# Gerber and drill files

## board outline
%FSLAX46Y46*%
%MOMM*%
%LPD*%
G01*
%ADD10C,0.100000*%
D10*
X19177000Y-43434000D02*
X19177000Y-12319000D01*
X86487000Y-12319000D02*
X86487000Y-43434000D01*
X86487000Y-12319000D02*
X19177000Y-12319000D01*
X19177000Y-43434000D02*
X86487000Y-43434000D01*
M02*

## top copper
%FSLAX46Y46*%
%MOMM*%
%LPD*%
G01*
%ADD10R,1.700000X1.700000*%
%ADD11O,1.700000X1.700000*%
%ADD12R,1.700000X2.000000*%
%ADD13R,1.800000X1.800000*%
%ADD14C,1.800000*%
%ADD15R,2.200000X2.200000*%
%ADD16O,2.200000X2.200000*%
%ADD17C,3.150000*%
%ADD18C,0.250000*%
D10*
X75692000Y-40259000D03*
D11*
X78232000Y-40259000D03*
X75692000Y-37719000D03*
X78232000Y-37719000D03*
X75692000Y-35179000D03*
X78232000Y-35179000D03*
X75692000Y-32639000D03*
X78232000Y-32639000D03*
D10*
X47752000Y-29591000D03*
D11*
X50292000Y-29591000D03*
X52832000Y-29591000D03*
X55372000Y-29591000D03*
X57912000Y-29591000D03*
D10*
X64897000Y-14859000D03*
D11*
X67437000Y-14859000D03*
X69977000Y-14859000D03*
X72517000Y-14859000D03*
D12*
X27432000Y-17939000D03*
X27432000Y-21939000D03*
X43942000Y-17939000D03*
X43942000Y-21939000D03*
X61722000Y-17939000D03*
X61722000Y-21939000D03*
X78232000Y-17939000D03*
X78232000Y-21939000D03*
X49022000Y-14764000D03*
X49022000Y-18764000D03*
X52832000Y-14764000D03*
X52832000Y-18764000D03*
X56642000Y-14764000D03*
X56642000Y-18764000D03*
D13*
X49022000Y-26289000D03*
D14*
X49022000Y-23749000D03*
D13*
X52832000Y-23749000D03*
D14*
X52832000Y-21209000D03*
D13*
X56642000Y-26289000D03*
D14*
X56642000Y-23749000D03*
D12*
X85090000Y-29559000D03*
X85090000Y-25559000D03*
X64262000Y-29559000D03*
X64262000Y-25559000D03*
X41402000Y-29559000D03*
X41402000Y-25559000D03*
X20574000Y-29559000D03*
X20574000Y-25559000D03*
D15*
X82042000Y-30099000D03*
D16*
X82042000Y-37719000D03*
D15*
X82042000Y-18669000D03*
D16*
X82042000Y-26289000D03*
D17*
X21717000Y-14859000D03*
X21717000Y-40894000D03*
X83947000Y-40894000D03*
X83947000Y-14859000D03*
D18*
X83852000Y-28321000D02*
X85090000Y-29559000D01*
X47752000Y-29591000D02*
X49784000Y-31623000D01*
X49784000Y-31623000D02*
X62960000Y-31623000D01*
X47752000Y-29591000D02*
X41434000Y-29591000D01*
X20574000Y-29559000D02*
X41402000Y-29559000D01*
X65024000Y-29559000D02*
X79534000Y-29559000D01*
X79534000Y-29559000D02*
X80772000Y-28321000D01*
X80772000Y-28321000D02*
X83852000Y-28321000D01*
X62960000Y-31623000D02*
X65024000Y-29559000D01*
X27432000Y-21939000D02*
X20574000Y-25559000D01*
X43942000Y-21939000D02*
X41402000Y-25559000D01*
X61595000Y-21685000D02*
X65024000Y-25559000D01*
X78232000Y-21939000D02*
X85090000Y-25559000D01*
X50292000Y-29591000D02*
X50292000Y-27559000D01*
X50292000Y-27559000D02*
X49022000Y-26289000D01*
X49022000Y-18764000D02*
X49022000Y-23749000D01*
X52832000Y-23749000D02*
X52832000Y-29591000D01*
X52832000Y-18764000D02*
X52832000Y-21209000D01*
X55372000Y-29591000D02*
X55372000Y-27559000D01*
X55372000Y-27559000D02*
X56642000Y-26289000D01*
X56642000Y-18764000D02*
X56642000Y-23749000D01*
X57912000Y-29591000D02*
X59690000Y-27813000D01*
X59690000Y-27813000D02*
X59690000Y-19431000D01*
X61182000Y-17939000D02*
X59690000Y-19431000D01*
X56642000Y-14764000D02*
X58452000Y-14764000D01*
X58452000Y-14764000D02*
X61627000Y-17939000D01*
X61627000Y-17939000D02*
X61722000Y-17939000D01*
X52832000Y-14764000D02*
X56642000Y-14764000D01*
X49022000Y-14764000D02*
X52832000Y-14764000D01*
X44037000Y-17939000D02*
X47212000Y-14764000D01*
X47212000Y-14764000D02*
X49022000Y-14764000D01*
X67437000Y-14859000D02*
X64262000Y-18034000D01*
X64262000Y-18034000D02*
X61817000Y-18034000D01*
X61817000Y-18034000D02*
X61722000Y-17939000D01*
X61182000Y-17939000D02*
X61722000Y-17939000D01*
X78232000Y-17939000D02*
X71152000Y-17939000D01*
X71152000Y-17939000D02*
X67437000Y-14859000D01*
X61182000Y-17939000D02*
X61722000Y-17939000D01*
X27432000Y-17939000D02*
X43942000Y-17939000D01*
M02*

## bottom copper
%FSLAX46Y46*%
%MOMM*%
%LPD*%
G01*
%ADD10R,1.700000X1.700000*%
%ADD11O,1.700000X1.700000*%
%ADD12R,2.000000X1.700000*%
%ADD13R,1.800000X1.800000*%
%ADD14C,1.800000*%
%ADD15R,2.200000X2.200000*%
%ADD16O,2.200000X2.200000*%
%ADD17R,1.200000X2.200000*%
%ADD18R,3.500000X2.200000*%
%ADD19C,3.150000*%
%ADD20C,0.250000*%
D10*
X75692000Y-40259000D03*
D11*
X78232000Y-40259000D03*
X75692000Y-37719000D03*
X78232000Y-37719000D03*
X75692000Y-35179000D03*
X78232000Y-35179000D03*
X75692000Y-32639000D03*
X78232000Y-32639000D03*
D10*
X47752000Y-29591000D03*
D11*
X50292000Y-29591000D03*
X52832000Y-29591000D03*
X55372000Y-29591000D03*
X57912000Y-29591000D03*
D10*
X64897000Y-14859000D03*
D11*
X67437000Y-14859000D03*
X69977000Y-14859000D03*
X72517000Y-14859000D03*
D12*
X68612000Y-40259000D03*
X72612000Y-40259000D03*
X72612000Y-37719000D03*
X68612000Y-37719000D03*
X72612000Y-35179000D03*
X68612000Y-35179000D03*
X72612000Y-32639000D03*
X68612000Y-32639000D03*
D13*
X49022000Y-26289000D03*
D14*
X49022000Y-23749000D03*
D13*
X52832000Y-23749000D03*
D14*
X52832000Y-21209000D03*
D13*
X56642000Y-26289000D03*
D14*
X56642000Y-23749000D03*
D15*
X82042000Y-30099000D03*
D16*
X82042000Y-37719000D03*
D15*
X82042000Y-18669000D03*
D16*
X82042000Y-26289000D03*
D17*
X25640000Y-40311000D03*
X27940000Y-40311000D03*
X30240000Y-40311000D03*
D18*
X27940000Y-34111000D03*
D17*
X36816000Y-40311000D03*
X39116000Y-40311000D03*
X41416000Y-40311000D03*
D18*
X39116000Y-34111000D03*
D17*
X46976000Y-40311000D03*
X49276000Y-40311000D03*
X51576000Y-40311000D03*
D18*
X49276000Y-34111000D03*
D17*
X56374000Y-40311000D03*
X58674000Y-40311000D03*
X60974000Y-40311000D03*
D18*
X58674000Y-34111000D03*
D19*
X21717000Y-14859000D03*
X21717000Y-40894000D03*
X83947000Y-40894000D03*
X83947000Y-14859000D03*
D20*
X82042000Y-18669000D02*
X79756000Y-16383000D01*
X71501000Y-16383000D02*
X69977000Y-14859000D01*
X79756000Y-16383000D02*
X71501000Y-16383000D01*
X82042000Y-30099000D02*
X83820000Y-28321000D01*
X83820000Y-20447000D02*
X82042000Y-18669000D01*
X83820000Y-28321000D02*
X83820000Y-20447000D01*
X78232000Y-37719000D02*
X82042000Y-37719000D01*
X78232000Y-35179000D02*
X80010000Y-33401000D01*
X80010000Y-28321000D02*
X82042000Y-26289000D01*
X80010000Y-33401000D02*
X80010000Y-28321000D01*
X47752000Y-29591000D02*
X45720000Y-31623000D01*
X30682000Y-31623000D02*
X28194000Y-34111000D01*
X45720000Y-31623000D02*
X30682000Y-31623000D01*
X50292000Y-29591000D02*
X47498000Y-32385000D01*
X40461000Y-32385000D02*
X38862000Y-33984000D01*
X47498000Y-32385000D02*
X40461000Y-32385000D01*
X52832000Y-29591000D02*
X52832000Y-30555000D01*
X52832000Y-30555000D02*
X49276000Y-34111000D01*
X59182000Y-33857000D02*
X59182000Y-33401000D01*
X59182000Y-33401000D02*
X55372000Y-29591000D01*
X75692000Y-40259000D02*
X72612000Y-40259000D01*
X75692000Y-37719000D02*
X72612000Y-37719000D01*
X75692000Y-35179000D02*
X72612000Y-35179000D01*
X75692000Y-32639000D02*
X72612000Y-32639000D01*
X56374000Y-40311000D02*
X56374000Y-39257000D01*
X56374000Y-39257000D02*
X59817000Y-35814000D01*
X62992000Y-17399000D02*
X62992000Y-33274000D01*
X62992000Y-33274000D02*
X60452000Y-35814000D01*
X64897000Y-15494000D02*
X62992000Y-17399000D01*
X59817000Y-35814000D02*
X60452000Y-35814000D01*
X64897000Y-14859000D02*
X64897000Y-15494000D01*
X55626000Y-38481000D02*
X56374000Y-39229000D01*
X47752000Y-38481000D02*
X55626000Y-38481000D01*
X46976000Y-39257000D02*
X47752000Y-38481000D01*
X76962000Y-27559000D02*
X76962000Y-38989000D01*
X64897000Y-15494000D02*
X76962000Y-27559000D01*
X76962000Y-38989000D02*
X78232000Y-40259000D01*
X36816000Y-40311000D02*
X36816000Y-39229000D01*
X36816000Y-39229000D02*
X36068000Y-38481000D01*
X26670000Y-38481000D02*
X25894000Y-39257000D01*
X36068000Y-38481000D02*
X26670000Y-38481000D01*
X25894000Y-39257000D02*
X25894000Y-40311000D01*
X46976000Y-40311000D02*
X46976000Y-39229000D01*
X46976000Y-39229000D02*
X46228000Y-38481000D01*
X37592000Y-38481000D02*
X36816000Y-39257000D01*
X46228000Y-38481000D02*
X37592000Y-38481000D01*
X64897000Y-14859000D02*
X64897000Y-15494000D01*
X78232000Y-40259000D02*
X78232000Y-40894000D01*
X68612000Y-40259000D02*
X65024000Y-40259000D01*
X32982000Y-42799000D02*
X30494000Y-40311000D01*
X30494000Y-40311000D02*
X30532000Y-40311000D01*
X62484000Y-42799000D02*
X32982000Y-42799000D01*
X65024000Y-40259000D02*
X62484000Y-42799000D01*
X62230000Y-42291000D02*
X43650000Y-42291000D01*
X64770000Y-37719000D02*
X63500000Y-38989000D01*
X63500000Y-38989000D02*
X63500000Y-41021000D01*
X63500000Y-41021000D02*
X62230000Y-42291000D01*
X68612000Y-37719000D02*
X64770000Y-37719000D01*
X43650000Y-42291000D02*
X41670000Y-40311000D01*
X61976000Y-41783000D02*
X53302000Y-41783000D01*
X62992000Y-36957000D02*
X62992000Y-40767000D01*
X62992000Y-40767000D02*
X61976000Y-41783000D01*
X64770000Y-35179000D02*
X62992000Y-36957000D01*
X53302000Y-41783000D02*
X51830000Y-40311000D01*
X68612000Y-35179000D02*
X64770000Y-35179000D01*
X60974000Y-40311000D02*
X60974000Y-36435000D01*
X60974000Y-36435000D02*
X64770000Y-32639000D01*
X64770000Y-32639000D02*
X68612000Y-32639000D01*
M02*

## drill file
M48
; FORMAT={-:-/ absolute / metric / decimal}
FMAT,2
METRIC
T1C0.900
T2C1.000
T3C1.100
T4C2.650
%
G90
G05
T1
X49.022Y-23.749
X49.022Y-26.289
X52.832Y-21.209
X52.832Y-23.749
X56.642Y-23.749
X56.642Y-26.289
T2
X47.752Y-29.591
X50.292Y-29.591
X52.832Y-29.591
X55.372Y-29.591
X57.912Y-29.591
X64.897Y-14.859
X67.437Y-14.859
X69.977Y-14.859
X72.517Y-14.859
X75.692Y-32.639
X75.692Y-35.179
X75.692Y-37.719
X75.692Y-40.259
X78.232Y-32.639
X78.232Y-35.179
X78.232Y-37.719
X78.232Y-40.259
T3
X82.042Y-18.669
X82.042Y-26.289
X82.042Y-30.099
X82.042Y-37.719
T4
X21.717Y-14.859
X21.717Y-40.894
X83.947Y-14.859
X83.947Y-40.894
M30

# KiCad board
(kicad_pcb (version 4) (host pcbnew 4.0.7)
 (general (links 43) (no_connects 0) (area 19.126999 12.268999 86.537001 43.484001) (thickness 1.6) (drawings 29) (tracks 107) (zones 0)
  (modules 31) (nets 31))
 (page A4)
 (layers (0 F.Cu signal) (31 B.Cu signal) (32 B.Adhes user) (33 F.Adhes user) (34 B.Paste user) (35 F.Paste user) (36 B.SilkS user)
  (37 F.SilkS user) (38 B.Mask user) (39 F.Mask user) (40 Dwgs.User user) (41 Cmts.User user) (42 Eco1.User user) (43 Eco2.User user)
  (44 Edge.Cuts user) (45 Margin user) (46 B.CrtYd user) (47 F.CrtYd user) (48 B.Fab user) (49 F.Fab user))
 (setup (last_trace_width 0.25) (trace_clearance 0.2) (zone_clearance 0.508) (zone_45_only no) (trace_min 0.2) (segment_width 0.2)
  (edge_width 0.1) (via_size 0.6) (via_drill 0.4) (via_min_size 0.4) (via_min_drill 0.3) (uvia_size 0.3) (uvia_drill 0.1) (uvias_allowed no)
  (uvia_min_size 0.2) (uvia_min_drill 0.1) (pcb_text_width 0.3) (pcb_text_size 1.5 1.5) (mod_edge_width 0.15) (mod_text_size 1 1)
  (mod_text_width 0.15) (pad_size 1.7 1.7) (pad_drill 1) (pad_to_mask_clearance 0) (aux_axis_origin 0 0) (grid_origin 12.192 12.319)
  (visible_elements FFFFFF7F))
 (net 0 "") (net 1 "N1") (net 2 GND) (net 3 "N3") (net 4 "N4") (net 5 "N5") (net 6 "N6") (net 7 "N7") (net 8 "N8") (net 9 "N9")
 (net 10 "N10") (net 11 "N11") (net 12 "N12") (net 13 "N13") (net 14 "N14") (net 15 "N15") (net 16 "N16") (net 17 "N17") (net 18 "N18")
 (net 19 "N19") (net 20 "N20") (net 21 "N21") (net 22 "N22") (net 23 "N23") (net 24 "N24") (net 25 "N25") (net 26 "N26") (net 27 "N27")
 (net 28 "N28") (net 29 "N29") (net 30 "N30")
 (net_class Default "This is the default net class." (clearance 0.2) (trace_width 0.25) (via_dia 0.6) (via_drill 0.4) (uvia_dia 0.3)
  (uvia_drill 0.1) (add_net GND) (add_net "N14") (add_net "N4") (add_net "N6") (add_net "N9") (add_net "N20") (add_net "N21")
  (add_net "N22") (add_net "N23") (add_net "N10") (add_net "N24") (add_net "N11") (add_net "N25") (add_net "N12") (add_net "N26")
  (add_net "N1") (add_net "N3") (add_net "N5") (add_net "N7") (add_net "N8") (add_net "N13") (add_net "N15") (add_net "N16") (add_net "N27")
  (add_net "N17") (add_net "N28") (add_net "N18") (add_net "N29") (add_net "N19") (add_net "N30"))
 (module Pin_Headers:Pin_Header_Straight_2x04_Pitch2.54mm (layer B.Cu) (at 75.692 40.259)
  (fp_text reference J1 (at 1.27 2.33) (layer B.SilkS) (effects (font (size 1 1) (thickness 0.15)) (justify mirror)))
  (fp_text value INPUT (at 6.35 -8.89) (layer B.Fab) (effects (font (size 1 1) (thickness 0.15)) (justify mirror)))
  (pad 1 thru_hole rect (at 0 0) (size 1.7 1.7) (drill 1) (layers *.Cu *.Mask) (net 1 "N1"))
  (pad 2 thru_hole oval (at 2.54 0) (size 1.7 1.7) (drill 1) (layers *.Cu *.Mask) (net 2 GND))
  (pad 3 thru_hole oval (at 0 -2.54) (size 1.7 1.7) (drill 1) (layers *.Cu *.Mask) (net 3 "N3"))
  (pad 4 thru_hole oval (at 2.54 -2.54) (size 1.7 1.7) (drill 1) (layers *.Cu *.Mask) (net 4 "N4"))
  (pad 5 thru_hole oval (at 0 -5.08) (size 1.7 1.7) (drill 1) (layers *.Cu *.Mask) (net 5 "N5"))
  (pad 6 thru_hole oval (at 2.54 -5.08) (size 1.7 1.7) (drill 1) (layers *.Cu *.Mask) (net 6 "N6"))
  (pad 7 thru_hole oval (at 0 -7.62) (size 1.7 1.7) (drill 1) (layers *.Cu *.Mask) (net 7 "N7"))
  (pad 8 thru_hole oval (at 2.54 -7.62) (size 1.7 1.7) (drill 1) (layers *.Cu *.Mask) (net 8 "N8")))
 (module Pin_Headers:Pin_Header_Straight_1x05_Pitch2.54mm (layer B.Cu) (at 47.752 29.591 270)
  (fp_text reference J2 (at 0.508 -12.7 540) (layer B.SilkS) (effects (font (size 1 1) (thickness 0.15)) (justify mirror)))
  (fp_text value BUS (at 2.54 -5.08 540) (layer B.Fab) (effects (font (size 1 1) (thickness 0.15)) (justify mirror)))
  (pad 1 thru_hole rect (at 0 0 270) (size 1.7 1.7) (drill 1) (layers *.Cu *.Mask) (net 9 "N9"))
  (pad 2 thru_hole oval (at 0 -2.54 270) (size 1.7 1.7) (drill 1) (layers *.Cu *.Mask) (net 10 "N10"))
  (pad 3 thru_hole oval (at 0 -5.08 270) (size 1.7 1.7) (drill 1) (layers *.Cu *.Mask) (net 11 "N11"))
  (pad 4 thru_hole oval (at 0 -7.62 270) (size 1.7 1.7) (drill 1) (layers *.Cu *.Mask) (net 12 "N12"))
  (pad 5 thru_hole oval (at 0 -10.16 270) (size 1.7 1.7) (drill 1) (layers *.Cu *.Mask) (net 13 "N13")))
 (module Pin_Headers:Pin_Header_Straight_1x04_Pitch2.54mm (layer B.Cu) (at 64.897 14.859 270)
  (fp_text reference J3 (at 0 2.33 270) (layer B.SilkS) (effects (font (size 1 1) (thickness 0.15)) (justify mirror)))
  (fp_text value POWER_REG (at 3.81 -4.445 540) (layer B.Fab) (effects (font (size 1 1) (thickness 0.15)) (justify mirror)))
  (pad 1 thru_hole rect (at 0 0 270) (size 1.7 1.7) (drill 1) (layers *.Cu *.Mask) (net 2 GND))
  (pad 2 thru_hole oval (at 0 -2.54 270) (size 1.7 1.7) (drill 1) (layers *.Cu *.Mask) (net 13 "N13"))
  (pad 3 thru_hole oval (at 0 -5.08 270) (size 1.7 1.7) (drill 1) (layers *.Cu *.Mask) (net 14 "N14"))
  (pad 4 thru_hole oval (at 0 -7.62 270) (size 1.7 1.7) (drill 1) (layers *.Cu *.Mask) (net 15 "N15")))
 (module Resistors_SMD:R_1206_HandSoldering (layer B.Cu) (at 70.612 40.259)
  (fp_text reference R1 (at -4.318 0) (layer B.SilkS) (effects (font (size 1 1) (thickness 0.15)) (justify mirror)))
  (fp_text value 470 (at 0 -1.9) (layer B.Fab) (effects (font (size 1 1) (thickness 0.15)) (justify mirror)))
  (pad 1 smd rect (at -2 0) (size 2 1.7) (layers B.Cu B.Paste B.Mask) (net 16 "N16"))
  (pad 2 smd rect (at 2 0) (size 2 1.7) (layers B.Cu B.Paste B.Mask) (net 1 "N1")))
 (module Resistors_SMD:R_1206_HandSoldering (layer B.Cu) (at 70.612 37.719 180)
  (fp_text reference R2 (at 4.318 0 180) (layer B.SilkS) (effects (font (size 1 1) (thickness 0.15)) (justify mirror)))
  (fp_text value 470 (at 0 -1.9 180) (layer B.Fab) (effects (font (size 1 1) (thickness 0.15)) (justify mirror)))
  (pad 1 smd rect (at -2 0 180) (size 2 1.7) (layers B.Cu B.Paste B.Mask) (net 3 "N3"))
  (pad 2 smd rect (at 2 0 180) (size 2 1.7) (layers B.Cu B.Paste B.Mask) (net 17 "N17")))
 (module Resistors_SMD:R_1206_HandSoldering (layer B.Cu) (at 70.612 35.179 180)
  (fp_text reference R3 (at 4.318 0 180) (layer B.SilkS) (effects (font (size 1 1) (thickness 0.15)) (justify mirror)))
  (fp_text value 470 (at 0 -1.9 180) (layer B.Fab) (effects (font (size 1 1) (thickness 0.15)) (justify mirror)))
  (pad 1 smd rect (at -2 0 180) (size 2 1.7) (layers B.Cu B.Paste B.Mask) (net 5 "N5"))
  (pad 2 smd rect (at 2 0 180) (size 2 1.7) (layers B.Cu B.Paste B.Mask) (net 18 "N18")))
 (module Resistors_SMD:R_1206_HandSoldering (layer B.Cu) (at 70.612 32.639 180)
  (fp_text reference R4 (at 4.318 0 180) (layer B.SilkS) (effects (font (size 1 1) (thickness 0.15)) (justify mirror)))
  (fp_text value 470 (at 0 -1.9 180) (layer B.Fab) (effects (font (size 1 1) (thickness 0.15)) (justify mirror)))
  (pad 1 smd rect (at -2 0 180) (size 2 1.7) (layers B.Cu B.Paste B.Mask) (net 7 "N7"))
  (pad 2 smd rect (at 2 0 180) (size 2 1.7) (layers B.Cu B.Paste B.Mask) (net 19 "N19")))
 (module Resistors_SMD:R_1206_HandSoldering (layer F.Cu) (at 27.432 19.939 270)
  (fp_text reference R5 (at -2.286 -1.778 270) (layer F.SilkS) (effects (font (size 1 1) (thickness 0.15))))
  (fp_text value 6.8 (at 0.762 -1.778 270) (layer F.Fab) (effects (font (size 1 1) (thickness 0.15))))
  (pad 1 smd rect (at -2 0 270) (size 2 1.7) (layers F.Cu F.Paste F.Mask) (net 13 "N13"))
  (pad 2 smd rect (at 2 0 270) (size 2 1.7) (layers F.Cu F.Paste F.Mask) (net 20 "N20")))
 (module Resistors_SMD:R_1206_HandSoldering (layer F.Cu) (at 43.942 19.939 270)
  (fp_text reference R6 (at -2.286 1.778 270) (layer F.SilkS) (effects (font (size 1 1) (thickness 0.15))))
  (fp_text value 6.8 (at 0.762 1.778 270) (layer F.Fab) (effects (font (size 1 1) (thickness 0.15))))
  (pad 1 smd rect (at -2 0 270) (size 2 1.7) (layers F.Cu F.Paste F.Mask) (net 13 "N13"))
  (pad 2 smd rect (at 2 0 270) (size 2 1.7) (layers F.Cu F.Paste F.Mask) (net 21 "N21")))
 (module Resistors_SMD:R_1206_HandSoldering (layer F.Cu) (at 61.722 19.939 270)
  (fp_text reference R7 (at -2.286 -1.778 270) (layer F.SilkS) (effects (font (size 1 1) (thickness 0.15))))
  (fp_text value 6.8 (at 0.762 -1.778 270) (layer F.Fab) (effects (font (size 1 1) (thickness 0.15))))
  (pad 1 smd rect (at -2 0 270) (size 2 1.7) (layers F.Cu F.Paste F.Mask) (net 13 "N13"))
  (pad 2 smd rect (at 2 0 270) (size 2 1.7) (layers F.Cu F.Paste F.Mask) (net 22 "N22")))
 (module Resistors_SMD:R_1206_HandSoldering (layer F.Cu) (at 78.232 19.939 270)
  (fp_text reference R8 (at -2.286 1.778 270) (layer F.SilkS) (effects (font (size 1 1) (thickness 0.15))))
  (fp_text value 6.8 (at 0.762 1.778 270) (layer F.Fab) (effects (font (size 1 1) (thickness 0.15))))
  (pad 1 smd rect (at -2 0 270) (size 2 1.7) (layers F.Cu F.Paste F.Mask) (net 13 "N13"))
  (pad 2 smd rect (at 2 0 270) (size 2 1.7) (layers F.Cu F.Paste F.Mask) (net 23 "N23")))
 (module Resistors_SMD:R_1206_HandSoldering (layer F.Cu) (at 49.022 16.764 270)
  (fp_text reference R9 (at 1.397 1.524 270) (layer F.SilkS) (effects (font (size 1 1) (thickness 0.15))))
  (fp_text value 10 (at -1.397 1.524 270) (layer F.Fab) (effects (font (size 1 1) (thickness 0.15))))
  (pad 1 smd rect (at -2 0 270) (size 2 1.7) (layers F.Cu F.Paste F.Mask) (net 13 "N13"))
  (pad 2 smd rect (at 2 0 270) (size 2 1.7) (layers F.Cu F.Paste F.Mask) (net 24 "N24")))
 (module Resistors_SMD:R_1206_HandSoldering (layer F.Cu) (at 52.832 16.764 270)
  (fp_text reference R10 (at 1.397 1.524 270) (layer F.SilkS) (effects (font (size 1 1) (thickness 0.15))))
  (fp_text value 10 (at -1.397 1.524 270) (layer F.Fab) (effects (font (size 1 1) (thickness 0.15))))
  (pad 1 smd rect (at -2 0 270) (size 2 1.7) (layers F.Cu F.Paste F.Mask) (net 13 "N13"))
  (pad 2 smd rect (at 2 0 270) (size 2 1.7) (layers F.Cu F.Paste F.Mask) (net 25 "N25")))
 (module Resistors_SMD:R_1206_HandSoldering (layer F.Cu) (at 56.642 16.764 270)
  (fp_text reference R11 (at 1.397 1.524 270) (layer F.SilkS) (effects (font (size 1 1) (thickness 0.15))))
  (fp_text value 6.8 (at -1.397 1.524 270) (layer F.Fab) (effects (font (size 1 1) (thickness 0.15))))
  (pad 1 smd rect (at -2 0 270) (size 2 1.7) (layers F.Cu F.Paste F.Mask) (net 13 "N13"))
  (pad 2 smd rect (at 2 0 270) (size 2 1.7) (layers F.Cu F.Paste F.Mask) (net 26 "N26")))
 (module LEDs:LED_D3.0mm (layer F.Cu) (at 49.022 26.289 90)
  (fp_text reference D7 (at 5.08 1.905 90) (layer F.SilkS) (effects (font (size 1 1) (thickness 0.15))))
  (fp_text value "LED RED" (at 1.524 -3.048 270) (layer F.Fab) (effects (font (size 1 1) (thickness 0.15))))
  (pad 1 thru_hole rect (at 0 0 90) (size 1.8 1.8) (drill 0.9) (layers *.Cu *.Mask) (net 10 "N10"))
  (pad 2 thru_hole circle (at 2.54 0 90) (size 1.8 1.8) (drill 0.9) (layers *.Cu *.Mask) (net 24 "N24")))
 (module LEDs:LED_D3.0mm (layer F.Cu) (at 52.832 23.749 90)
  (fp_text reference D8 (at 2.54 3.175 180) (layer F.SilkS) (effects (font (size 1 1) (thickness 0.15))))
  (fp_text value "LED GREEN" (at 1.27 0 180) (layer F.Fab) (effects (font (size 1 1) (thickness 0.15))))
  (pad 1 thru_hole rect (at 0 0 90) (size 1.8 1.8) (drill 0.9) (layers *.Cu *.Mask) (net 11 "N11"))
  (pad 2 thru_hole circle (at 2.54 0 90) (size 1.8 1.8) (drill 0.9) (layers *.Cu *.Mask) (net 25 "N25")))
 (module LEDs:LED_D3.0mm (layer F.Cu) (at 56.642 26.289 90)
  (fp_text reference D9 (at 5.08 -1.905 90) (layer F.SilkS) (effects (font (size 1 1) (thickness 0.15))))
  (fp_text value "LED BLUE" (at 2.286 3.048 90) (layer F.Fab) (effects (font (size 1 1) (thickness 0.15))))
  (pad 1 thru_hole rect (at 0 0 90) (size 1.8 1.8) (drill 0.9) (layers *.Cu *.Mask) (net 12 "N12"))
  (pad 2 thru_hole circle (at 2.54 0 90) (size 1.8 1.8) (drill 0.9) (layers *.Cu *.Mask) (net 26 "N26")))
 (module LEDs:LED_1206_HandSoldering (layer F.Cu) (at 85.09 27.559 90)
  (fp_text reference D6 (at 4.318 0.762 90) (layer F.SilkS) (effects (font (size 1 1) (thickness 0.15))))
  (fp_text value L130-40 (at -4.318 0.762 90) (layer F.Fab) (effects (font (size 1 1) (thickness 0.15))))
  (pad 1 smd rect (at -2 0 90) (size 2 1.7) (layers F.Cu F.Paste F.Mask) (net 9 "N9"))
  (pad 2 smd rect (at 2 0 90) (size 2 1.7) (layers F.Cu F.Paste F.Mask) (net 23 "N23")))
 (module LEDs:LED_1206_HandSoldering (layer F.Cu) (at 64.262 27.559 90)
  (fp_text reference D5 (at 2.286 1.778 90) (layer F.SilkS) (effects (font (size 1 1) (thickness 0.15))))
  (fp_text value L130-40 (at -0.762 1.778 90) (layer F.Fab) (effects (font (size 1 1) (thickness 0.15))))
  (pad 1 smd rect (at -2 0 90) (size 2 1.7) (layers F.Cu F.Paste F.Mask) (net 9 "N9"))
  (pad 2 smd rect (at 2 0 90) (size 2 1.7) (layers F.Cu F.Paste F.Mask) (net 22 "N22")))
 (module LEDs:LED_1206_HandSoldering (layer F.Cu) (at 41.402 27.559 90)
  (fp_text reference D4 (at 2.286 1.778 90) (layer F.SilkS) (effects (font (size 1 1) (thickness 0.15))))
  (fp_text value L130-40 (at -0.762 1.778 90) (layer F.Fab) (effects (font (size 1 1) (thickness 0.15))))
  (pad 1 smd rect (at -2 0 90) (size 2 1.7) (layers F.Cu F.Paste F.Mask) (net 9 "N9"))
  (pad 2 smd rect (at 2 0 90) (size 2 1.7) (layers F.Cu F.Paste F.Mask) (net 21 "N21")))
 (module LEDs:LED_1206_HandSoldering (layer F.Cu) (at 20.574 27.559 90)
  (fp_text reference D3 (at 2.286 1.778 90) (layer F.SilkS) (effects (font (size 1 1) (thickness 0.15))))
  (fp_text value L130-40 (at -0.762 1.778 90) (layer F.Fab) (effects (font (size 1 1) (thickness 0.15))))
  (pad 1 smd rect (at -2 0 90) (size 2 1.7) (layers F.Cu F.Paste F.Mask) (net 9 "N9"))
  (pad 2 smd rect (at 2 0 90) (size 2 1.7) (layers F.Cu F.Paste F.Mask) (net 20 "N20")))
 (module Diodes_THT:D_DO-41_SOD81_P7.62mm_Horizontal (layer B.Cu) (at 82.042 30.099 270)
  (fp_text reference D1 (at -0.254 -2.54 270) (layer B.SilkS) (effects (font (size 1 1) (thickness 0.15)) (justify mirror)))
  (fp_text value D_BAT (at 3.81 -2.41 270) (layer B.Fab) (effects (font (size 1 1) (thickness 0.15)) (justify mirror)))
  (pad 1 thru_hole rect (at 0 0 270) (size 2.2 2.2) (drill 1.1) (layers *.Cu *.Mask) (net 14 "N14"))
  (pad 2 thru_hole oval (at 7.62 0 270) (size 2.2 2.2) (drill 1.1) (layers *.Cu *.Mask) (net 4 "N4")))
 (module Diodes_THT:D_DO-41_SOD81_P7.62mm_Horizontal (layer B.Cu) (at 82.042 18.669 270)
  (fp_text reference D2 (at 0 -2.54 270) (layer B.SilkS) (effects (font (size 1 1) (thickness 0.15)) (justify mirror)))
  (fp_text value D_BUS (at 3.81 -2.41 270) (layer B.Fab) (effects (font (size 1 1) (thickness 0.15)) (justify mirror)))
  (pad 1 thru_hole rect (at 0 0 270) (size 2.2 2.2) (drill 1.1) (layers *.Cu *.Mask) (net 14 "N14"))
  (pad 2 thru_hole oval (at 7.62 0 270) (size 2.2 2.2) (drill 1.1) (layers *.Cu *.Mask) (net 6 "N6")))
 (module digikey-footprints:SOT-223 (layer B.Cu) (at 27.94 37.211 180)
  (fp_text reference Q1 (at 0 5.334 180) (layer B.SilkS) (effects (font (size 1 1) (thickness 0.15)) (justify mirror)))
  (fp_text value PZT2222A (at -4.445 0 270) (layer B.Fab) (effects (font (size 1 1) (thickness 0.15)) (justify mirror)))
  (pad 3 smd rect (at 2.3 -3.1 180) (size 1.2 2.2) (layers B.Cu B.Paste B.Mask) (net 2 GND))
  (pad 2 smd rect (at 0 -3.1 180) (size 1.2 2.2) (layers B.Cu B.Paste B.Mask) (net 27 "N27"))
  (pad 1 smd rect (at -2.3 -3.1 180) (size 1.2 2.2) (layers B.Cu B.Paste B.Mask) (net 16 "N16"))
  (pad 4 smd rect (at 0 3.1 180) (size 3.5 2.2) (layers B.Cu B.Paste B.Mask) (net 9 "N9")))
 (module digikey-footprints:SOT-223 (layer B.Cu) (at 39.116 37.211 180)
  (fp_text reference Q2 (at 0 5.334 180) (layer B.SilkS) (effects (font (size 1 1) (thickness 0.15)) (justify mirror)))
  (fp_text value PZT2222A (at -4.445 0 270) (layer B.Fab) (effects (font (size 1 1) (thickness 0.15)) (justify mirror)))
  (pad 3 smd rect (at 2.3 -3.1 180) (size 1.2 2.2) (layers B.Cu B.Paste B.Mask) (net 2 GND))
  (pad 2 smd rect (at 0 -3.1 180) (size 1.2 2.2) (layers B.Cu B.Paste B.Mask) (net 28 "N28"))
  (pad 1 smd rect (at -2.3 -3.1 180) (size 1.2 2.2) (layers B.Cu B.Paste B.Mask) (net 17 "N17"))
  (pad 4 smd rect (at 0 3.1 180) (size 3.5 2.2) (layers B.Cu B.Paste B.Mask) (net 10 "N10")))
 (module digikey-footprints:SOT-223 (layer B.Cu) (at 49.276 37.211 180)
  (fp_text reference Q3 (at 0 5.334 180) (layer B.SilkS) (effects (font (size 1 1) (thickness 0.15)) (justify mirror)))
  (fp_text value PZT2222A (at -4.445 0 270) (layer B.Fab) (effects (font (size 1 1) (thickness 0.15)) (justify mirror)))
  (pad 3 smd rect (at 2.3 -3.1 180) (size 1.2 2.2) (layers B.Cu B.Paste B.Mask) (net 2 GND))
  (pad 2 smd rect (at 0 -3.1 180) (size 1.2 2.2) (layers B.Cu B.Paste B.Mask) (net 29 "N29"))
  (pad 1 smd rect (at -2.3 -3.1 180) (size 1.2 2.2) (layers B.Cu B.Paste B.Mask) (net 18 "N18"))
  (pad 4 smd rect (at 0 3.1 180) (size 3.5 2.2) (layers B.Cu B.Paste B.Mask) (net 11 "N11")))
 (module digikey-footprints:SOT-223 (layer B.Cu) (at 58.674 37.211 180)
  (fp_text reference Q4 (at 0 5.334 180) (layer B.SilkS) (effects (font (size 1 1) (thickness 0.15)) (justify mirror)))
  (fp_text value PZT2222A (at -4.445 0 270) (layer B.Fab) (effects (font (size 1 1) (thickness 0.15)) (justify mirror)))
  (pad 3 smd rect (at 2.3 -3.1 180) (size 1.2 2.2) (layers B.Cu B.Paste B.Mask) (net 2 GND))
  (pad 2 smd rect (at 0 -3.1 180) (size 1.2 2.2) (layers B.Cu B.Paste B.Mask) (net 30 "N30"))
  (pad 1 smd rect (at -2.3 -3.1 180) (size 1.2 2.2) (layers B.Cu B.Paste B.Mask) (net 19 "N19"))
  (pad 4 smd rect (at 0 3.1 180) (size 3.5 2.2) (layers B.Cu B.Paste B.Mask) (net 12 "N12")))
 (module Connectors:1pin (layer F.Cu) (at 21.717 14.859)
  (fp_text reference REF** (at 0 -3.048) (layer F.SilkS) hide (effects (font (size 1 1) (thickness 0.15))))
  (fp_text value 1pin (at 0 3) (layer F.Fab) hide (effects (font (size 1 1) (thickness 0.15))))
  (pad 1 thru_hole circle (at 0 0) (size 3.15 3.15) (drill 2.65) (layers *.Cu *.Mask)))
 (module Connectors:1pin (layer F.Cu) (at 21.717 40.894)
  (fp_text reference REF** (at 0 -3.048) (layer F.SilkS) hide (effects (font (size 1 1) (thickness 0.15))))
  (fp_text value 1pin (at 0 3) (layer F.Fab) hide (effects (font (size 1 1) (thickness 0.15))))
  (pad 1 thru_hole circle (at 0 0) (size 3.15 3.15) (drill 2.65) (layers *.Cu *.Mask)))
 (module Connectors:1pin (layer F.Cu) (at 83.947 40.894)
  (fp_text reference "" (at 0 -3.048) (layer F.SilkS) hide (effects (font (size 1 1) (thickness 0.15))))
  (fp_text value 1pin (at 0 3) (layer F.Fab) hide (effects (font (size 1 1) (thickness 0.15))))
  (pad 1 thru_hole circle (at 0 0) (size 3.15 3.15) (drill 2.65) (layers *.Cu *.Mask)))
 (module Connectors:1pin (layer F.Cu) (at 83.947 14.859)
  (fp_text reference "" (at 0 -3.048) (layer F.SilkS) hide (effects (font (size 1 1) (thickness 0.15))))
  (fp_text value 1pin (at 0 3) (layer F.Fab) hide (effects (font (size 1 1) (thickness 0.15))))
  (pad 1 thru_hole circle (at 0 0) (size 3.15 3.15) (drill 2.65) (layers *.Cu *.Mask)))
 (gr_line (start 19.177 43.434) (end 19.177 12.319) (angle 90) (layer Edge.Cuts) (width 0.1))
 (gr_line (start 86.487 12.319) (end 86.487 43.434) (angle 90) (layer Edge.Cuts) (width 0.1))
 (gr_line (start 86.487 12.319) (end 19.177 12.319) (angle 90) (layer Edge.Cuts) (width 0.1))
 (gr_line (start 19.177 43.434) (end 86.487 43.434) (angle 90) (layer Edge.Cuts) (width 0.1))
 (segment (start 82.042 18.669) (end 79.756 16.383) (width 0.25) (layer B.Cu) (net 14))
 (segment (start 71.501 16.383) (end 69.977 14.859) (width 0.25) (layer B.Cu) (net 14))
 (segment (start 79.756 16.383) (end 71.501 16.383) (width 0.25) (layer B.Cu) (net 14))
 (segment (start 82.042 30.099) (end 83.82 28.321) (width 0.25) (layer B.Cu) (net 14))
 (segment (start 83.82 20.447) (end 82.042 18.669) (width 0.25) (layer B.Cu) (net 14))
 (segment (start 83.82 28.321) (end 83.82 20.447) (width 0.25) (layer B.Cu) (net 14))
 (segment (start 78.232 37.719) (end 82.042 37.719) (width 0.25) (layer B.Cu) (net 4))
 (segment (start 78.232 35.179) (end 80.01 33.401) (width 0.25) (layer B.Cu) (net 6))
 (segment (start 80.01 28.321) (end 82.042 26.289) (width 0.25) (layer B.Cu) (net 6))
 (segment (start 80.01 33.401) (end 80.01 28.321) (width 0.25) (layer B.Cu) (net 6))
 (segment (start 83.852 28.321) (end 85.09 29.559) (width 0.25) (layer F.Cu) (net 9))
 (segment (start 47.752 29.591) (end 49.784 31.623) (width 0.25) (layer F.Cu) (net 9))
 (segment (start 49.784 31.623) (end 62.96 31.623) (width 0.25) (layer F.Cu) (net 9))
 (segment (start 47.752 29.591) (end 45.72 31.623) (width 0.25) (layer B.Cu) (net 9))
 (segment (start 30.682 31.623) (end 28.194 34.111) (width 0.25) (layer B.Cu) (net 9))
 (segment (start 45.72 31.623) (end 30.682 31.623) (width 0.25) (layer B.Cu) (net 9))
 (segment (start 47.752 29.591) (end 41.434 29.591) (width 0.25) (layer F.Cu) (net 9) (status 20))
 (segment (start 20.574 29.559) (end 41.402 29.559) (width 0.25) (layer F.Cu) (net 9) (status 20))
 (segment (start 65.024 29.559) (end 79.534 29.559) (width 0.25) (layer F.Cu) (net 9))
 (segment (start 79.534 29.559) (end 80.772 28.321) (width 0.25) (layer F.Cu) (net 9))
 (segment (start 80.772 28.321) (end 83.852 28.321) (width 0.25) (layer F.Cu) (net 9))
 (segment (start 62.96 31.623) (end 65.024 29.559) (width 0.25) (layer F.Cu) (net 9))
 (segment (start 27.432 21.939) (end 20.574 25.559) (width 0.25) (layer F.Cu) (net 20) (status 20))
 (segment (start 43.942 21.939) (end 41.402 25.559) (width 0.25) (layer F.Cu) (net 21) (status 20))
 (segment (start 61.595 21.685) (end 65.024 25.559) (width 0.25) (layer F.Cu) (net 22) (status 20))
 (segment (start 78.232 21.939) (end 85.09 25.559) (width 0.25) (layer F.Cu) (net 23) (status 20))
 (segment (start 50.292 29.591) (end 47.498 32.385) (width 0.25) (layer B.Cu) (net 10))
 (segment (start 40.461 32.385) (end 38.862 33.984) (width 0.25) (layer B.Cu) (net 10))
 (segment (start 47.498 32.385) (end 40.461 32.385) (width 0.25) (layer B.Cu) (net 10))
 (segment (start 50.292 29.591) (end 50.292 27.559) (width 0.25) (layer F.Cu) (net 10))
 (segment (start 50.292 27.559) (end 49.022 26.289) (width 0.25) (layer F.Cu) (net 10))
 (segment (start 49.022 18.764) (end 49.022 23.749) (width 0.25) (layer F.Cu) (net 24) (status 10))
 (segment (start 52.832 29.591) (end 52.832 30.555) (width 0.25) (layer B.Cu) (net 11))
 (segment (start 52.832 30.555) (end 49.276 34.111) (width 0.25) (layer B.Cu) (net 11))
 (segment (start 52.832 23.749) (end 52.832 29.591) (width 0.25) (layer F.Cu) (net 11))
 (segment (start 52.832 18.764) (end 52.832 21.209) (width 0.25) (layer F.Cu) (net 25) (status 10))
 (segment (start 59.182 33.857) (end 59.182 33.401) (width 0.25) (layer B.Cu) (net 12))
 (segment (start 59.182 33.401) (end 55.372 29.591) (width 0.25) (layer B.Cu) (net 12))
 (segment (start 55.372 29.591) (end 55.372 27.559) (width 0.25) (layer F.Cu) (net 12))
 (segment (start 55.372 27.559) (end 56.642 26.289) (width 0.25) (layer F.Cu) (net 12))
 (segment (start 56.642 18.764) (end 56.642 23.749) (width 0.25) (layer F.Cu) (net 26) (status 10))
 (segment (start 75.692 40.259) (end 72.612 40.259) (width 0.25) (layer B.Cu) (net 1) (status 10))
 (segment (start 75.692 37.719) (end 72.612 37.719) (width 0.25) (layer B.Cu) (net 3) (status 10))
 (segment (start 75.692 35.179) (end 72.612 35.179) (width 0.25) (layer B.Cu) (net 5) (status 10))
 (segment (start 75.692 32.639) (end 72.612 32.639) (width 0.25) (layer B.Cu) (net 7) (status 10))
 (segment (start 56.374 40.311) (end 56.374 39.257) (width 0.25) (layer B.Cu) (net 2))
 (segment (start 56.374 39.257) (end 59.817 35.814) (width 0.25) (layer B.Cu) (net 2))
 (segment (start 62.992 17.399) (end 62.992 33.274) (width 0.25) (layer B.Cu) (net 2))
 (segment (start 62.992 33.274) (end 60.452 35.814) (width 0.25) (layer B.Cu) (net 2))
 (segment (start 64.897 15.494) (end 62.992 17.399) (width 0.25) (layer B.Cu) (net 2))
 (segment (start 59.817 35.814) (end 60.452 35.814) (width 0.25) (layer B.Cu) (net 2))
 (segment (start 64.897 14.859) (end 64.897 15.494) (width 0.25) (layer B.Cu) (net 2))
 (segment (start 55.626 38.481) (end 56.374 39.229) (width 0.25) (layer B.Cu) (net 2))
 (segment (start 47.752 38.481) (end 55.626 38.481) (width 0.25) (layer B.Cu) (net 2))
 (segment (start 46.976 39.257) (end 47.752 38.481) (width 0.25) (layer B.Cu) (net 2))
 (segment (start 76.962 27.559) (end 76.962 38.989) (width 0.25) (layer B.Cu) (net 2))
 (segment (start 64.897 15.494) (end 76.962 27.559) (width 0.25) (layer B.Cu) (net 2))
 (segment (start 76.962 38.989) (end 78.232 40.259) (width 0.25) (layer B.Cu) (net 2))
 (segment (start 36.816 40.311) (end 36.816 39.229) (width 0.25) (layer B.Cu) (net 2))
 (segment (start 36.816 39.229) (end 36.068 38.481) (width 0.25) (layer B.Cu) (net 2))
 (segment (start 26.67 38.481) (end 25.894 39.257) (width 0.25) (layer B.Cu) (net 2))
 (segment (start 36.068 38.481) (end 26.67 38.481) (width 0.25) (layer B.Cu) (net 2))
 (segment (start 25.894 39.257) (end 25.894 40.311) (width 0.25) (layer B.Cu) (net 2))
 (segment (start 46.976 40.311) (end 46.976 39.229) (width 0.25) (layer B.Cu) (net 2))
 (segment (start 46.976 39.229) (end 46.228 38.481) (width 0.25) (layer B.Cu) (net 2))
 (segment (start 37.592 38.481) (end 36.816 39.257) (width 0.25) (layer B.Cu) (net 2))
 (segment (start 46.228 38.481) (end 37.592 38.481) (width 0.25) (layer B.Cu) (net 2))
 (segment (start 64.897 14.859) (end 64.897 15.494) (width 0.25) (layer B.Cu) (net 2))
 (segment (start 78.232 40.259) (end 78.232 40.894) (width 0.25) (layer B.Cu) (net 2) (status 30))
 (segment (start 57.912 29.591) (end 59.69 27.813) (width 0.25) (layer F.Cu) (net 13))
 (segment (start 59.69 27.813) (end 59.69 19.431) (width 0.25) (layer F.Cu) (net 13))
 (segment (start 61.182 17.939) (end 59.69 19.431) (width 0.25) (layer F.Cu) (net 13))
 (segment (start 56.642 14.764) (end 58.452 14.764) (width 0.25) (layer F.Cu) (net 13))
 (segment (start 58.452 14.764) (end 61.627 17.939) (width 0.25) (layer F.Cu) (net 13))
 (segment (start 61.627 17.939) (end 61.722 17.939) (width 0.25) (layer F.Cu) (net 13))
 (segment (start 52.832 14.764) (end 56.642 14.764) (width 0.25) (layer F.Cu) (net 13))
 (segment (start 49.022 14.764) (end 52.832 14.764) (width 0.25) (layer F.Cu) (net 13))
 (segment (start 44.037 17.939) (end 47.212 14.764) (width 0.25) (layer F.Cu) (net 13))
 (segment (start 47.212 14.764) (end 49.022 14.764) (width 0.25) (layer F.Cu) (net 13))
 (segment (start 67.437 14.859) (end 64.262 18.034) (width 0.25) (layer F.Cu) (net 13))
 (segment (start 64.262 18.034) (end 61.817 18.034) (width 0.25) (layer F.Cu) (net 13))
 (segment (start 61.817 18.034) (end 61.722 17.939) (width 0.25) (layer F.Cu) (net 13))
 (segment (start 61.182 17.939) (end 61.722 17.939) (width 0.25) (layer F.Cu) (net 13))
 (segment (start 78.232 17.939) (end 71.152 17.939) (width 0.25) (layer F.Cu) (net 13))
 (segment (start 71.152 17.939) (end 67.437 14.859) (width 0.25) (layer F.Cu) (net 13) (status 20))
 (segment (start 61.182 17.939) (end 61.722 17.939) (width 0.25) (layer F.Cu) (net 13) (status 30))
 (segment (start 27.432 17.939) (end 43.942 17.939) (width 0.25) (layer F.Cu) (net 13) (status 10))
 (segment (start 68.612 40.259) (end 65.024 40.259) (width 0.25) (layer B.Cu) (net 16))
 (segment (start 32.982 42.799) (end 30.494 40.311) (width 0.25) (layer B.Cu) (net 16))
 (segment (start 30.494 40.311) (end 30.532 40.311) (width 0.25) (layer B.Cu) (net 16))
 (segment (start 62.484 42.799) (end 32.982 42.799) (width 0.25) (layer B.Cu) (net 16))
 (segment (start 65.024 40.259) (end 62.484 42.799) (width 0.25) (layer B.Cu) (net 16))
 (segment (start 62.23 42.291) (end 43.65 42.291) (width 0.25) (layer B.Cu) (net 17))
 (segment (start 64.77 37.719) (end 63.5 38.989) (width 0.25) (layer B.Cu) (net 17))
 (segment (start 63.5 38.989) (end 63.5 41.021) (width 0.25) (layer B.Cu) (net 17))
 (segment (start 63.5 41.021) (end 62.23 42.291) (width 0.25) (layer B.Cu) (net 17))
 (segment (start 68.612 37.719) (end 64.77 37.719) (width 0.25) (layer B.Cu) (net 17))
 (segment (start 43.65 42.291) (end 41.67 40.311) (width 0.25) (layer B.Cu) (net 17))
 (segment (start 61.976 41.783) (end 53.302 41.783) (width 0.25) (layer B.Cu) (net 18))
 (segment (start 62.992 36.957) (end 62.992 40.767) (width 0.25) (layer B.Cu) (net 18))
 (segment (start 62.992 40.767) (end 61.976 41.783) (width 0.25) (layer B.Cu) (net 18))
 (segment (start 64.77 35.179) (end 62.992 36.957) (width 0.25) (layer B.Cu) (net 18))
 (segment (start 53.302 41.783) (end 51.83 40.311) (width 0.25) (layer B.Cu) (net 18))
 (segment (start 68.612 35.179) (end 64.77 35.179) (width 0.25) (layer B.Cu) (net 18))
 (segment (start 60.974 40.311) (end 60.974 36.435) (width 0.25) (layer B.Cu) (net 19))
 (segment (start 60.974 36.435) (end 64.77 32.639) (width 0.25) (layer B.Cu) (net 19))
 (segment (start 64.77 32.639) (end 68.612 32.639) (width 0.25) (layer B.Cu) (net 19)))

